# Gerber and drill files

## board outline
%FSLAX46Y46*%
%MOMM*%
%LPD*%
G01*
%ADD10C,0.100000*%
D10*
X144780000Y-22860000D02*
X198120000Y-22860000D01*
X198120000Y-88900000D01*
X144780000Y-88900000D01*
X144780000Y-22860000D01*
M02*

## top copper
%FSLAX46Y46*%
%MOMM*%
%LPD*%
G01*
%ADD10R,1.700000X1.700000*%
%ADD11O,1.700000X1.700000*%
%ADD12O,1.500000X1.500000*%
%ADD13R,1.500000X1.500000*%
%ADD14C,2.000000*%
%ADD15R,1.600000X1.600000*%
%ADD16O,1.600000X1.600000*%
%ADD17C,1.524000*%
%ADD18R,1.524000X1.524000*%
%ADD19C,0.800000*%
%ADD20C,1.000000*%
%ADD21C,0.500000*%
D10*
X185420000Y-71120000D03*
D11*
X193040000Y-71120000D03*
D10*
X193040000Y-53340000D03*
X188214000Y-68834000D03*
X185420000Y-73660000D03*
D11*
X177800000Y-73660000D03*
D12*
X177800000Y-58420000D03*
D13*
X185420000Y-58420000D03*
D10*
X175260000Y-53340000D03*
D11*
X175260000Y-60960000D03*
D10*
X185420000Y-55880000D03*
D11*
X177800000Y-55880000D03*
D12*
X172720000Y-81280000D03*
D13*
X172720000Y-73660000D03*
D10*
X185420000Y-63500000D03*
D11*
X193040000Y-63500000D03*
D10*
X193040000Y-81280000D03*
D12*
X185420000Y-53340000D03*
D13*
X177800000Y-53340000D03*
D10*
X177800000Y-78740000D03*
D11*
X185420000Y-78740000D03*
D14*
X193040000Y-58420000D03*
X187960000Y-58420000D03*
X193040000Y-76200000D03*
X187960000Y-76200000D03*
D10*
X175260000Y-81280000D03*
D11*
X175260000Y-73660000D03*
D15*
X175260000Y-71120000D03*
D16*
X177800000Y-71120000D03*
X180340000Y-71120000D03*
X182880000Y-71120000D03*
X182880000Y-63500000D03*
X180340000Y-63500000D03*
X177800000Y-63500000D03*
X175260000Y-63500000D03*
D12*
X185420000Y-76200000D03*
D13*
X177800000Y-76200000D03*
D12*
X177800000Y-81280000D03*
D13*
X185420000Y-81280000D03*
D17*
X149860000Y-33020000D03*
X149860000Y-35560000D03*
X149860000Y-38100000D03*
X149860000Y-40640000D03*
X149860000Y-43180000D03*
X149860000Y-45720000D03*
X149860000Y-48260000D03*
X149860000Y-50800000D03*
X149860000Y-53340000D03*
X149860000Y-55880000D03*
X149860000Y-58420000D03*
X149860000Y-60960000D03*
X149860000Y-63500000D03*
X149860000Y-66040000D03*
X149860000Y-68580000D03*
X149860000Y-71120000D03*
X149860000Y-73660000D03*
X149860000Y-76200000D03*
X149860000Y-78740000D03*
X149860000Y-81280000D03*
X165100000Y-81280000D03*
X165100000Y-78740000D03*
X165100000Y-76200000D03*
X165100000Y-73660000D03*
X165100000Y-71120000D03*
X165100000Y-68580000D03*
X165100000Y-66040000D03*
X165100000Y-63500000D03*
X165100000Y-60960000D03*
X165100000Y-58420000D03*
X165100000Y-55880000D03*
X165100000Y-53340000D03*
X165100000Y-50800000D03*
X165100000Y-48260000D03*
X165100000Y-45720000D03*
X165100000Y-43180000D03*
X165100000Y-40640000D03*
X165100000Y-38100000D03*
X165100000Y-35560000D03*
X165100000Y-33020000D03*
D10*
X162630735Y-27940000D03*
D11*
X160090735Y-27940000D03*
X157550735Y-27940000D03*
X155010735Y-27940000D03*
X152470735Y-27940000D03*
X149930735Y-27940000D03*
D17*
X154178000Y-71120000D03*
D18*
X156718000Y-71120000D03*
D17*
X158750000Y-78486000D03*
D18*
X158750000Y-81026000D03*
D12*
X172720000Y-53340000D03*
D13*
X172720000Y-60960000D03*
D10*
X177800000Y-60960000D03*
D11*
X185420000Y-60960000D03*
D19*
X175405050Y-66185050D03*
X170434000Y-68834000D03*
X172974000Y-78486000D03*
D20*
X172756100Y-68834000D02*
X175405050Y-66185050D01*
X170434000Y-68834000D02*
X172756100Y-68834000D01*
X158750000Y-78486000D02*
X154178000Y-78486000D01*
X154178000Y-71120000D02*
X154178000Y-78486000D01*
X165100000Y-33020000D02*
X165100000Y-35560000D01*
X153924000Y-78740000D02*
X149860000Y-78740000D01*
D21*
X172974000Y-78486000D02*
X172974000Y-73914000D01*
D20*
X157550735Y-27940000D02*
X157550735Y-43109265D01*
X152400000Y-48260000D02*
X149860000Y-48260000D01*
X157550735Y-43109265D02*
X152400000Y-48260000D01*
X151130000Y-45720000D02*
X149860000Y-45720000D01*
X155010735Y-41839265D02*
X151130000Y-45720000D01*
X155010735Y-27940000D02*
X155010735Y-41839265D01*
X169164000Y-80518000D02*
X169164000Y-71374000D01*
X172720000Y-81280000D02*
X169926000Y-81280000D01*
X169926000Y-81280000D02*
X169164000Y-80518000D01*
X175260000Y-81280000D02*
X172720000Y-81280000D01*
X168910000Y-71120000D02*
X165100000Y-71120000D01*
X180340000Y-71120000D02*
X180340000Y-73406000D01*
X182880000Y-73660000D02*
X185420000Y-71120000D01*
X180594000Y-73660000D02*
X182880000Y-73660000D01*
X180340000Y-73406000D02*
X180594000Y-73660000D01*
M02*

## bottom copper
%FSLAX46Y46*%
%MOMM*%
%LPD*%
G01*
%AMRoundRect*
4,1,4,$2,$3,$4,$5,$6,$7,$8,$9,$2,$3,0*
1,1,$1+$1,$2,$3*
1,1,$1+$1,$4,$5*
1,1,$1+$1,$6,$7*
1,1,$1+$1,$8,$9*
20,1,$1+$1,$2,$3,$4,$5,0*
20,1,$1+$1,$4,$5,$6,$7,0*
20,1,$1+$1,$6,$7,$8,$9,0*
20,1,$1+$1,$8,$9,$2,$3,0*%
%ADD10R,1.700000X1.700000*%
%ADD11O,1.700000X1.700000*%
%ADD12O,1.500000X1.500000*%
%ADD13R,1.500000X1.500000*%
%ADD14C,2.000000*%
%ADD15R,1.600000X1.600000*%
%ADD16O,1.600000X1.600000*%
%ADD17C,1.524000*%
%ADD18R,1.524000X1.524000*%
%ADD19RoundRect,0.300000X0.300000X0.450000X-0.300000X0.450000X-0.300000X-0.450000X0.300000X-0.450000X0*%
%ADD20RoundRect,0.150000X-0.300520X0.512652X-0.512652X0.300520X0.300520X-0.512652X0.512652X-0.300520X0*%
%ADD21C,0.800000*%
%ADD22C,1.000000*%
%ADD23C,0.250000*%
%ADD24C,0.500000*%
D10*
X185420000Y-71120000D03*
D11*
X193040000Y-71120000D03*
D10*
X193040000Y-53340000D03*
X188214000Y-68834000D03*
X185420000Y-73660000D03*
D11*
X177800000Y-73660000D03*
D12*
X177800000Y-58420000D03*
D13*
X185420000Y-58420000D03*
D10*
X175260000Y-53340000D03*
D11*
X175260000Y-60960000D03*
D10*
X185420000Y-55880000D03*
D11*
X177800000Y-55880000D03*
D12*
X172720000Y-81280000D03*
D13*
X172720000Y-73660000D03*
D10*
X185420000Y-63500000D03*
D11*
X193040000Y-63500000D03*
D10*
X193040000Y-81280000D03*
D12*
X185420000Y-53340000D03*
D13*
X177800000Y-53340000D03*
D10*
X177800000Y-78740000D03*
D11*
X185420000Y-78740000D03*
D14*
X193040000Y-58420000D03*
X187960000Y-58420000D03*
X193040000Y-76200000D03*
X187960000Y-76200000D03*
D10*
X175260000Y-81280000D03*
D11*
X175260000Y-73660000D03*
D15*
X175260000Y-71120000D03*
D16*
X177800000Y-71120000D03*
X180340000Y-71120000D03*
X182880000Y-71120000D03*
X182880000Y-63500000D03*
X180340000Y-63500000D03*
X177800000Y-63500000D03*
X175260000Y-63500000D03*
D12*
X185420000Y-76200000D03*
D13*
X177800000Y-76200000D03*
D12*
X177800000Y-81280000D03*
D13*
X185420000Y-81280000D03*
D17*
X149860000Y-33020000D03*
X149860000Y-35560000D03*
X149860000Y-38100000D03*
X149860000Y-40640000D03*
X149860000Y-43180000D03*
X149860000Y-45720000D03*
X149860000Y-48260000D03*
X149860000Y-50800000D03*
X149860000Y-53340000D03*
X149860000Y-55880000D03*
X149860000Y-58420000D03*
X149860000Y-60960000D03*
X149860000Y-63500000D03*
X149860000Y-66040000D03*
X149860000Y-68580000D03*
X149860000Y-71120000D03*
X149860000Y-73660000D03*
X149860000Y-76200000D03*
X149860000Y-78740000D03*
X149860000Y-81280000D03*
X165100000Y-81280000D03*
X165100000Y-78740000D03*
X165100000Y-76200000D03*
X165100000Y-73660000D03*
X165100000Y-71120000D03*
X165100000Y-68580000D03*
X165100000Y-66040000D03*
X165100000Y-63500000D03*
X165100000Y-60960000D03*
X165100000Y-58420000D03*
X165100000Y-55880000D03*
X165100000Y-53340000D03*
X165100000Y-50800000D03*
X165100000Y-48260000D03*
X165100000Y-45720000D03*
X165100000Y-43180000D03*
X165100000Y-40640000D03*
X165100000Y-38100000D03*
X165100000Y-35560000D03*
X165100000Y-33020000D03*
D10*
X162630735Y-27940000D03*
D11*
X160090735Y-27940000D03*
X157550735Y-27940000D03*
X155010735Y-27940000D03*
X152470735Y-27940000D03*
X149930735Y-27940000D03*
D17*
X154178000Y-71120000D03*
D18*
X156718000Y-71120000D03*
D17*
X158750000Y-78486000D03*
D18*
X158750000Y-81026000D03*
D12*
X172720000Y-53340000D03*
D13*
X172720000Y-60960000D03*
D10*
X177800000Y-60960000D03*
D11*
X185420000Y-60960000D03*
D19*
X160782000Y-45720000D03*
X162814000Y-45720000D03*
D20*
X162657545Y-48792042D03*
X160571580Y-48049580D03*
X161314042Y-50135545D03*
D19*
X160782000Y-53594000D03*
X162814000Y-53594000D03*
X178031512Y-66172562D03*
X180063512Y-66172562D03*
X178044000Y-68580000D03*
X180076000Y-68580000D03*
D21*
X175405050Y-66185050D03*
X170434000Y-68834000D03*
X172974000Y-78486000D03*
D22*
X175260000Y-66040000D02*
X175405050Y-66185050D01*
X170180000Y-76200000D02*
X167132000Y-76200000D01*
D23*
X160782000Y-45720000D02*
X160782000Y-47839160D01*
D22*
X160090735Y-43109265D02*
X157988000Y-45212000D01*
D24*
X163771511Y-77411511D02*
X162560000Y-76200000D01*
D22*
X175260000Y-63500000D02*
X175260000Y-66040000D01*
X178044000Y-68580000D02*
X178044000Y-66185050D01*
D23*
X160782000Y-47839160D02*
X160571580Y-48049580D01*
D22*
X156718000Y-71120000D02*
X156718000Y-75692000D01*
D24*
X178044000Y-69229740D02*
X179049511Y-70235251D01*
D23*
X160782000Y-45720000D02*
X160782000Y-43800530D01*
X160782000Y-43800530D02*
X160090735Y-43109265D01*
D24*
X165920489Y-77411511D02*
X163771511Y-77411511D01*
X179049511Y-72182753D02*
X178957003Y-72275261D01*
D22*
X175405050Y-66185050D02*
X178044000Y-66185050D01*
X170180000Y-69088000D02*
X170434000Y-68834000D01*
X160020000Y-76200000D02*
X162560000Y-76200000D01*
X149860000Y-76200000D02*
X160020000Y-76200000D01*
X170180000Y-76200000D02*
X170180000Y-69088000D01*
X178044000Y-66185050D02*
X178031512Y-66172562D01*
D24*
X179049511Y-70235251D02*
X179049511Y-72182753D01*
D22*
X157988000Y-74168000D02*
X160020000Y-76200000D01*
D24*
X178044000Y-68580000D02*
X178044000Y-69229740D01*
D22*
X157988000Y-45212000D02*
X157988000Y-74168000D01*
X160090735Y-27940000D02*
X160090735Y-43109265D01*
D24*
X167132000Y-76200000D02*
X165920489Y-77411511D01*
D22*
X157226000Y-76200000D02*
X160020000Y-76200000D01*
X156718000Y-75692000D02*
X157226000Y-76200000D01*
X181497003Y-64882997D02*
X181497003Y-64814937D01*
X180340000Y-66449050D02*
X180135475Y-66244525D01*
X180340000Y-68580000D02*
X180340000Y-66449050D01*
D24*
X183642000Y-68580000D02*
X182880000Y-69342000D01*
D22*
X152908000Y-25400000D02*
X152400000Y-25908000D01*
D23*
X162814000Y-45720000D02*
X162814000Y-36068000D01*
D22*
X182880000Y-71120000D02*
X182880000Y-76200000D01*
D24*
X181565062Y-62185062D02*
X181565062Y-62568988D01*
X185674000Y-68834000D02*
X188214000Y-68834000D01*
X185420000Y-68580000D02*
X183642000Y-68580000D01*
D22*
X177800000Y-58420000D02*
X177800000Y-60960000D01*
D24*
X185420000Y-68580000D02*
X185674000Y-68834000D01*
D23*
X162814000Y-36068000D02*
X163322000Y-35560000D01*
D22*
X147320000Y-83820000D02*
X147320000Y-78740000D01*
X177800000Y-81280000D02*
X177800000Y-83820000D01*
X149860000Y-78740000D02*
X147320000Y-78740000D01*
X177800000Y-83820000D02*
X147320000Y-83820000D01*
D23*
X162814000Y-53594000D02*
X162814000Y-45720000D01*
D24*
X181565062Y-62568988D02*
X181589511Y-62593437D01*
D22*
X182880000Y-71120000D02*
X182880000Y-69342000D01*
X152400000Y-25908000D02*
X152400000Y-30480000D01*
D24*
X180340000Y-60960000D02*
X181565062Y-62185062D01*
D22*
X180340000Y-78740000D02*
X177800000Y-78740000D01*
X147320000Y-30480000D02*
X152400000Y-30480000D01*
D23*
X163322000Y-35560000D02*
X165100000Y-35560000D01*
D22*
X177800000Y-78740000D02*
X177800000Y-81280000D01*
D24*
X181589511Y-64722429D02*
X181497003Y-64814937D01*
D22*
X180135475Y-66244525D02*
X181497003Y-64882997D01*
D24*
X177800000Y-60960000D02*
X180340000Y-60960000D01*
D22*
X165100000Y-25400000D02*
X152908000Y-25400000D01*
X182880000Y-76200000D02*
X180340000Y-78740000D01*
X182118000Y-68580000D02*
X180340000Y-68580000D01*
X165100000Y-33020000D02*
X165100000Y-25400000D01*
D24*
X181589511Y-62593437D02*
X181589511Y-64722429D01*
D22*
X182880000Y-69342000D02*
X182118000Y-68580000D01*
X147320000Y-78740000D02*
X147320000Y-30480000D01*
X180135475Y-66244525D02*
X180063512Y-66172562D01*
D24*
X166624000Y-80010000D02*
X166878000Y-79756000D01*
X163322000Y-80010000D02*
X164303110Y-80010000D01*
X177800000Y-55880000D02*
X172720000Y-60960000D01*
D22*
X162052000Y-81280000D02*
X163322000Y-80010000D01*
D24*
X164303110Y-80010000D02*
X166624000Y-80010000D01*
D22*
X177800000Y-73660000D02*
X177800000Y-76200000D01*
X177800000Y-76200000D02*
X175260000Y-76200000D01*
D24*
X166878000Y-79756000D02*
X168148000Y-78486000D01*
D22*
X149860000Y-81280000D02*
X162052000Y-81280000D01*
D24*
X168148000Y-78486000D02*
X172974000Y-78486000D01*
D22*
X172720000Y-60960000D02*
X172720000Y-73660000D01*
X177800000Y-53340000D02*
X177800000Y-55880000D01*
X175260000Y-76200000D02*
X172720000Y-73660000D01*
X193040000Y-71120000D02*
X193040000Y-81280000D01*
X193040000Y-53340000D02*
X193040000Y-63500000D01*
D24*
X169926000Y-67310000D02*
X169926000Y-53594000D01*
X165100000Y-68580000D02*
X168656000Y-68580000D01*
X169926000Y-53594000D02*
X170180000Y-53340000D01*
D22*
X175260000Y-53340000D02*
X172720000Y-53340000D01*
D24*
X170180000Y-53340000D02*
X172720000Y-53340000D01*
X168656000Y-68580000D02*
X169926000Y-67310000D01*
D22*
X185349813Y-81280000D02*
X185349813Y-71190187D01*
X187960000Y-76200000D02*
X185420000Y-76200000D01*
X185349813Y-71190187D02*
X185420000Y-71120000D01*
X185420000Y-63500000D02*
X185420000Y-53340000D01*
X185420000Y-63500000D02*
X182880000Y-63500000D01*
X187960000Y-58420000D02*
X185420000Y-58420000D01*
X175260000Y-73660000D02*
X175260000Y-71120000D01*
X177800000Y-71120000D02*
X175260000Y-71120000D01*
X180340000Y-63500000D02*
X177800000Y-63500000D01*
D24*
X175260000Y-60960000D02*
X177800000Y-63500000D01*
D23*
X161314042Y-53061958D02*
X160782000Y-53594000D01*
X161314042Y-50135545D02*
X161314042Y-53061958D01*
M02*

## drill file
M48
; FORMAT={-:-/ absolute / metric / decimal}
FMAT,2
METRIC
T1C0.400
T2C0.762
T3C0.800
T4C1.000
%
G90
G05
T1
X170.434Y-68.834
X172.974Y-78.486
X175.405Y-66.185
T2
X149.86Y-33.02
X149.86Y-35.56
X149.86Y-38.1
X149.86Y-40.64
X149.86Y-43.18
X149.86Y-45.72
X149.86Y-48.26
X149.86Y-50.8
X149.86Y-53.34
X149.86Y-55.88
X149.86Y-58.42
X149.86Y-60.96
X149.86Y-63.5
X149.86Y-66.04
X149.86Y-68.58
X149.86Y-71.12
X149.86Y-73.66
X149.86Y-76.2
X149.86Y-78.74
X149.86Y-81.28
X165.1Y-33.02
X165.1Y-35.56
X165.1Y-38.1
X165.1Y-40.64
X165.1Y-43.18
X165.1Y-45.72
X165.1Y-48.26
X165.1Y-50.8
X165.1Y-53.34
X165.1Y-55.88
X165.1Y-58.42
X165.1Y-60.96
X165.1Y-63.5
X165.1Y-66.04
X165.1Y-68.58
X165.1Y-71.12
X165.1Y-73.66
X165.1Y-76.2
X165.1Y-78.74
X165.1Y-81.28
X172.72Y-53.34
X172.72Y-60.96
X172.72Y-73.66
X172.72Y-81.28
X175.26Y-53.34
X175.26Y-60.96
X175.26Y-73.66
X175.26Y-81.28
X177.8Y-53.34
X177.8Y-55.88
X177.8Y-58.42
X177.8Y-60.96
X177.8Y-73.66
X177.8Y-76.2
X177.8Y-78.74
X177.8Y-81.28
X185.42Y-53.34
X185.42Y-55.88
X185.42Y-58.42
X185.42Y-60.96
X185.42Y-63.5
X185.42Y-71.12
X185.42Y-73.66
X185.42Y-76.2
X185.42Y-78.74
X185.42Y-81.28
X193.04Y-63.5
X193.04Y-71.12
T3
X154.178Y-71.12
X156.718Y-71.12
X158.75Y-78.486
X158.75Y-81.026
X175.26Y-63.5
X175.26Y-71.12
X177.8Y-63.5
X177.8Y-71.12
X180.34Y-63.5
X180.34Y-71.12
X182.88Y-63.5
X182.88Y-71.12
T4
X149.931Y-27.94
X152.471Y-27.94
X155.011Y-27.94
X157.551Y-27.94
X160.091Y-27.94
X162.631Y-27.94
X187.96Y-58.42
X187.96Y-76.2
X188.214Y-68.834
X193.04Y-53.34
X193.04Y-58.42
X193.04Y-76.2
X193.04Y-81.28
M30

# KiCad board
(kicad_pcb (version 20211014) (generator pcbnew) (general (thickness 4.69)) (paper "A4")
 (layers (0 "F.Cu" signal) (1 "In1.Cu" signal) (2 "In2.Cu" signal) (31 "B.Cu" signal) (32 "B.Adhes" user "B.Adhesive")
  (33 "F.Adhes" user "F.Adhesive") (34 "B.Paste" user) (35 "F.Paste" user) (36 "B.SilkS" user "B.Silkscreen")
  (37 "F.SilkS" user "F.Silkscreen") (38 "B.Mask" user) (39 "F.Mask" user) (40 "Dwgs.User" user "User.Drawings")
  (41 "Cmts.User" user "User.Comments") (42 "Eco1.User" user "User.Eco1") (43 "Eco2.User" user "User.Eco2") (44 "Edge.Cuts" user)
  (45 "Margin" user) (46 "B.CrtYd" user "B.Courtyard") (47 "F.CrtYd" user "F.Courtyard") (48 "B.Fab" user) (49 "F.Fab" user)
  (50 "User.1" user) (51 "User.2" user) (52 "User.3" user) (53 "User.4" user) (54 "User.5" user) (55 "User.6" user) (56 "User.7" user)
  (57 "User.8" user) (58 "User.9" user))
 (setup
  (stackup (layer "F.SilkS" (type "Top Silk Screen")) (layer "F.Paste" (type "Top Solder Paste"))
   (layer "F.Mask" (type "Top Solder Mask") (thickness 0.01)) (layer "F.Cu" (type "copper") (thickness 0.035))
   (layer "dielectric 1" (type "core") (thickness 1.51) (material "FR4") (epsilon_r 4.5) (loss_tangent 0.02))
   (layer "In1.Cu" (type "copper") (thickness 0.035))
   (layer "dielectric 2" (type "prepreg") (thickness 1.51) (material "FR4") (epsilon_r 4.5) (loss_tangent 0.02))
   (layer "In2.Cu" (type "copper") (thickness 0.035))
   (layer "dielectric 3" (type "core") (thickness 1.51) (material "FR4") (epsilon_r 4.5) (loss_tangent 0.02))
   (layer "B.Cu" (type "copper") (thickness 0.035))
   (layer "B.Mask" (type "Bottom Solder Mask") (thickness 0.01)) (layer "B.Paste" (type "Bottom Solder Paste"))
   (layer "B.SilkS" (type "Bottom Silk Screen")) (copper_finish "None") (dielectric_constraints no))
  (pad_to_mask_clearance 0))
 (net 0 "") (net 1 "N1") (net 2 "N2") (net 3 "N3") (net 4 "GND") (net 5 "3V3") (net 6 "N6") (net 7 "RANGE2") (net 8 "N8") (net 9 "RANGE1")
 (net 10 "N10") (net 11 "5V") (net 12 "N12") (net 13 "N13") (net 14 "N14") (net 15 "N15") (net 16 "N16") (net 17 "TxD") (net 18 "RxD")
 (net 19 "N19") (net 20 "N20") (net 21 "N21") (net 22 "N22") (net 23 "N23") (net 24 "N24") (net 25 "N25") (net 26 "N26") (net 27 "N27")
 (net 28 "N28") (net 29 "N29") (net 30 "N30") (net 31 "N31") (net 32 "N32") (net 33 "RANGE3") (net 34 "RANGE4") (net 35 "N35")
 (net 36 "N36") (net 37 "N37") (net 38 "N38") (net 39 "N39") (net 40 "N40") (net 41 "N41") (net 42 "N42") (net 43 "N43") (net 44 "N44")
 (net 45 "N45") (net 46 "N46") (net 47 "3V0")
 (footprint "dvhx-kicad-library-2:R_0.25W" (layer "F.Cu") (at 185.42 71.12)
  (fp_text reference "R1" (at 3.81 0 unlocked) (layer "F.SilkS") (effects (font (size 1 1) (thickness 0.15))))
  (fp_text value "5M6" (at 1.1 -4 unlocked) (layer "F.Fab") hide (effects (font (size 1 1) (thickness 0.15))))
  (pad "1" thru_hole rect (at 0 0 90) (size 1.7 1.7) (drill 0.762) (layers *.Cu *.Mask) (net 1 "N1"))
  (pad "2" thru_hole oval (at 7.62 0 90) (size 1.7 1.7) (drill 0.762) (layers *.Cu *.Mask) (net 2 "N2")))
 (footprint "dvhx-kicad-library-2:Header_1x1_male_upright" (layer "F.Cu") (at 193.04 53.34 -90)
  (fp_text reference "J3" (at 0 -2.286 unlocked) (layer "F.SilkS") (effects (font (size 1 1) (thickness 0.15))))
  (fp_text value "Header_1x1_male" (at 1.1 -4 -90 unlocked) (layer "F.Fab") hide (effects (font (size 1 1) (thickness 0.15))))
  (pad "1" thru_hole rect (at 0 0 270) (size 1.7 1.7) (drill 1) (layers *.Cu *.Mask) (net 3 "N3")))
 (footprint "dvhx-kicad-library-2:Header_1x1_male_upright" (layer "F.Cu") (at 188.214 68.834)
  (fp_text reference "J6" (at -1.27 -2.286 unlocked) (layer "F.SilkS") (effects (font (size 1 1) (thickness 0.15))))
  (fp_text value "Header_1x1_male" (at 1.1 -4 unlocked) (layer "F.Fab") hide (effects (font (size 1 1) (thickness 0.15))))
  (pad "1" thru_hole rect (at 0 0) (size 1.7 1.7) (drill 1) (layers *.Cu *.Mask) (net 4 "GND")))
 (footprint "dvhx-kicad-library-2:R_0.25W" (layer "F.Cu") (at 185.42 73.66 180)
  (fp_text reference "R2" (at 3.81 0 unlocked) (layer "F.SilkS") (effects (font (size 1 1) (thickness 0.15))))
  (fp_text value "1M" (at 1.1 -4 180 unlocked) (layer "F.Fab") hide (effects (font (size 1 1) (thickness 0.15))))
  (pad "1" thru_hole rect (at 0 0 270) (size 1.7 1.7) (drill 0.762) (layers *.Cu *.Mask) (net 1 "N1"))
  (pad "2" thru_hole oval (at 7.62 0 270) (size 1.7 1.7) (drill 0.762) (layers *.Cu *.Mask) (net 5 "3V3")))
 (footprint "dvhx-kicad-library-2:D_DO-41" (layer "F.Cu") (at 181.61 58.42 90)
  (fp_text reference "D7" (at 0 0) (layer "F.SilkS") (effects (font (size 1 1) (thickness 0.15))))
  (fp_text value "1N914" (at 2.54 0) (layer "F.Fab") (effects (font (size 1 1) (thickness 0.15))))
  (pad "A" thru_hole oval (at 0 -3.81 180) (size 1.5 1.5) (drill 0.762) (layers *.Cu *.Mask) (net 4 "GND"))
  (pad "K" thru_hole rect (at 0 3.81 180) (size 1.5 1.5) (drill 0.762) (layers *.Cu *.Mask) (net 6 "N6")))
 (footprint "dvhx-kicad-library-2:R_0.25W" (layer "F.Cu") (at 175.26 53.34 -90)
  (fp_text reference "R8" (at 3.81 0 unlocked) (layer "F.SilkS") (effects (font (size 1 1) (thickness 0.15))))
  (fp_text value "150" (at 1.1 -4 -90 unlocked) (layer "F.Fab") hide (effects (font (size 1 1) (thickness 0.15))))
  (pad "1" thru_hole rect (at 0 0) (size 1.7 1.7) (drill 0.762) (layers *.Cu *.Mask) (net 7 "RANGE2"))
  (pad "2" thru_hole oval (at 7.62 0) (size 1.7 1.7) (drill 0.762) (layers *.Cu *.Mask) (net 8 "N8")))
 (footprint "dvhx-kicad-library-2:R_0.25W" (layer "F.Cu") (at 185.42 55.88 180)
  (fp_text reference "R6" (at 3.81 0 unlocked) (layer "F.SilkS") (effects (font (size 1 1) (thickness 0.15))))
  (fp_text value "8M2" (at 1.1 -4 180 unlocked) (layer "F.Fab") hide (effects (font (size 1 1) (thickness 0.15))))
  (pad "1" thru_hole rect (at 0 0 270) (size 1.7 1.7) (drill 0.762) (layers *.Cu *.Mask) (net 6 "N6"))
  (pad "2" thru_hole oval (at 7.62 0 270) (size 1.7 1.7) (drill 0.762) (layers *.Cu *.Mask) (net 5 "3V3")))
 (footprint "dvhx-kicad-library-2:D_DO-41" (layer "F.Cu") (at 172.72 77.47 180)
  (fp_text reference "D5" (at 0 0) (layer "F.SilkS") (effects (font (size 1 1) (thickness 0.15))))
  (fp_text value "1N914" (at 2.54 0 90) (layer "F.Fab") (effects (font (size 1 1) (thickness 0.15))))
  (pad "A" thru_hole oval (at 0 -3.81 270) (size 1.5 1.5) (drill 0.762) (layers *.Cu *.Mask) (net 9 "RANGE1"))
  (pad "K" thru_hole rect (at 0 3.81 270) (size 1.5 1.5) (drill 0.762) (layers *.Cu *.Mask) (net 5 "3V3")))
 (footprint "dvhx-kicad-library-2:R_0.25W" (layer "F.Cu") (at 185.42 63.5)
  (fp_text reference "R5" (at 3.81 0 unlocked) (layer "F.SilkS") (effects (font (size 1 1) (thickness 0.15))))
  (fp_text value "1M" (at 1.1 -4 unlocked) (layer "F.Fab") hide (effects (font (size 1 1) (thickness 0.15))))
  (pad "1" thru_hole rect (at 0 0 90) (size 1.7 1.7) (drill 0.762) (layers *.Cu *.Mask) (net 6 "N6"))
  (pad "2" thru_hole oval (at 7.62 0 90) (size 1.7 1.7) (drill 0.762) (layers *.Cu *.Mask) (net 3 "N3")))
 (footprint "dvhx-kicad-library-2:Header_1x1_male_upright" (layer "F.Cu") (at 193.04 81.28 -90)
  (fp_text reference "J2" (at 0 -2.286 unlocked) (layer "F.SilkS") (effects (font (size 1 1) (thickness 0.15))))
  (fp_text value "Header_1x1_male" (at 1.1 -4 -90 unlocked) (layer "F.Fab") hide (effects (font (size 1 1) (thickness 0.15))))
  (pad "1" thru_hole rect (at 0 0 270) (size 1.7 1.7) (drill 1) (layers *.Cu *.Mask) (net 2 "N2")))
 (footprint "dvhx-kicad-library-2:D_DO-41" (layer "F.Cu") (at 181.61 53.34 -90)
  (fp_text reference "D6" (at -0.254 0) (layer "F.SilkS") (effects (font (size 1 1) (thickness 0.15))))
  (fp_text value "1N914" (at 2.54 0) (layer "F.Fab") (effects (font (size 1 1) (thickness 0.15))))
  (pad "A" thru_hole oval (at 0 -3.81) (size 1.5 1.5) (drill 0.762) (layers *.Cu *.Mask) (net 6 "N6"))
  (pad "K" thru_hole rect (at 0 3.81) (size 1.5 1.5) (drill 0.762) (layers *.Cu *.Mask) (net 5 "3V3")))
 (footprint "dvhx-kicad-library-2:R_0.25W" (layer "F.Cu") (at 177.8 78.74)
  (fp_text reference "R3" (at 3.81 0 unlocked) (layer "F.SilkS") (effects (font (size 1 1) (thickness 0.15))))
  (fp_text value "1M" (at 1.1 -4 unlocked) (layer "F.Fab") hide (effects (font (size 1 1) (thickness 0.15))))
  (pad "1" thru_hole rect (at 0 0 90) (size 1.7 1.7) (drill 0.762) (layers *.Cu *.Mask) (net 4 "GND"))
  (pad "2" thru_hole oval (at 7.62 0 90) (size 1.7 1.7) (drill 0.762) (layers *.Cu *.Mask) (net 1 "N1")))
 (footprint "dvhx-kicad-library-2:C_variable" (layer "F.Cu") (at 193.04 58.42 -90)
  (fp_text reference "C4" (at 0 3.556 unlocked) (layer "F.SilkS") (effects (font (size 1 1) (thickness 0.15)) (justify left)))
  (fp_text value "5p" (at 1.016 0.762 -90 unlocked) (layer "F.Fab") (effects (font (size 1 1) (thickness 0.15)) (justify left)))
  (pad "1" thru_hole circle (at 0 0 270) (size 2 2) (drill 1) (layers *.Cu *.Mask) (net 3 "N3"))
  (pad "2" thru_hole circle (at 0 5.08 270) (size 2 2) (drill 1) (layers *.Cu *.Mask) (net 6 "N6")))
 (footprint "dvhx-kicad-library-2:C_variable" (layer "F.Cu") (at 193.04 76.2 -90)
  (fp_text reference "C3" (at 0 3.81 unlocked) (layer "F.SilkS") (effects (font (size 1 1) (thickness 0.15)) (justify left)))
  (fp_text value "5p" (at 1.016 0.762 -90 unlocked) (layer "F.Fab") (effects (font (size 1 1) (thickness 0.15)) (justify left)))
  (pad "1" thru_hole circle (at 0 0 270) (size 2 2) (drill 1) (layers *.Cu *.Mask) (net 2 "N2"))
  (pad "2" thru_hole circle (at 0 5.08 270) (size 2 2) (drill 1) (layers *.Cu *.Mask) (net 1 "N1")))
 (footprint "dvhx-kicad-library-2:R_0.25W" (layer "F.Cu") (at 175.26 81.28 90)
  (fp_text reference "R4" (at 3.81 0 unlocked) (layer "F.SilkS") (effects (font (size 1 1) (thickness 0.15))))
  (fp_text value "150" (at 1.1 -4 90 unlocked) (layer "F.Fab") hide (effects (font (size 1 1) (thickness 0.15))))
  (pad "1" thru_hole rect (at 0 0 180) (size 1.7 1.7) (drill 0.762) (layers *.Cu *.Mask) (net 9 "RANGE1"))
  (pad "2" thru_hole oval (at 7.62 0 180) (size 1.7 1.7) (drill 0.762) (layers *.Cu *.Mask) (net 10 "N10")))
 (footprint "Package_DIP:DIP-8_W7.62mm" (layer "F.Cu") (at 175.26 71.12 90)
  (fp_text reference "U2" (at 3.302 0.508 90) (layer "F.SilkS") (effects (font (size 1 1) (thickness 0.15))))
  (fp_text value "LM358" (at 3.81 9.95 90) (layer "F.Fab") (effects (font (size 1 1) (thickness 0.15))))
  (pad "1" thru_hole rect (at 0 0 90) (size 1.6 1.6) (drill 0.8) (layers *.Cu *.Mask) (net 10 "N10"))
  (pad "2" thru_hole oval (at 0 2.54 90) (size 1.6 1.6) (drill 0.8) (layers *.Cu *.Mask) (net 10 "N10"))
  (pad "3" thru_hole oval (at 0 5.08 90) (size 1.6 1.6) (drill 0.8) (layers *.Cu *.Mask) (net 1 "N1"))
  (pad "4" thru_hole oval (at 0 7.62 90) (size 1.6 1.6) (drill 0.8) (layers *.Cu *.Mask) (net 4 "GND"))
  (pad "5" thru_hole oval (at 7.62 7.62 90) (size 1.6 1.6) (drill 0.8) (layers *.Cu *.Mask) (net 6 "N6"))
  (pad "6" thru_hole oval (at 7.62 5.08 90) (size 1.6 1.6) (drill 0.8) (layers *.Cu *.Mask) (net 8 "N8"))
  (pad "7" thru_hole oval (at 7.62 2.54 90) (size 1.6 1.6) (drill 0.8) (layers *.Cu *.Mask) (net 8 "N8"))
  (pad "8" thru_hole oval (at 7.62 0 90) (size 1.6 1.6) (drill 0.8) (layers *.Cu *.Mask) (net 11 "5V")))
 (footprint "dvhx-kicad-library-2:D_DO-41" (layer "F.Cu") (at 181.61 76.2 -90)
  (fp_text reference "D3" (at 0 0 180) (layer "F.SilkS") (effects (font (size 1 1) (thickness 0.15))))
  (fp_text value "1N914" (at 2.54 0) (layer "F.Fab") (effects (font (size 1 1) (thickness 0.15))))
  (pad "A" thru_hole oval (at 0 -3.81) (size 1.5 1.5) (drill 0.762) (layers *.Cu *.Mask) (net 1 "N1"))
  (pad "K" thru_hole rect (at 0 3.81) (size 1.5 1.5) (drill 0.762) (layers *.Cu *.Mask) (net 5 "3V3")))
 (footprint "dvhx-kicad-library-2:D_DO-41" (layer "F.Cu") (at 181.61 81.28 90)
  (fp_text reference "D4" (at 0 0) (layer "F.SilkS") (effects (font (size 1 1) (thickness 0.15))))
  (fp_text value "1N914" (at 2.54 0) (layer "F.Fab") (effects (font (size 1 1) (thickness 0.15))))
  (pad "A" thru_hole oval (at 0 -3.81 180) (size 1.5 1.5) (drill 0.762) (layers *.Cu *.Mask) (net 4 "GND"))
  (pad "K" thru_hole rect (at 0 3.81 180) (size 1.5 1.5) (drill 0.762) (layers *.Cu *.Mask) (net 1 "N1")))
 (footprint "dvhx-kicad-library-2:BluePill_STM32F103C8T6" (layer "F.Cu") (at 149.86 33.02)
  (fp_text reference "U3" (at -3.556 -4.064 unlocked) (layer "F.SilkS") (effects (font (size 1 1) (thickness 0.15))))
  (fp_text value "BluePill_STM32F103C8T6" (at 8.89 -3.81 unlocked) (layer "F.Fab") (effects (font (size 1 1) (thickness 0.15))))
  (pad "1" thru_hole circle (at 0 0) (size 1.524 1.524) (drill 0.762) (layers *.Cu *.Mask) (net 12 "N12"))
  (pad "2" thru_hole circle (at 0 2.54) (size 1.524 1.524) (drill 0.762) (layers *.Cu *.Mask) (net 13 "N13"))
  (pad "3" thru_hole circle (at 0 5.08) (size 1.524 1.524) (drill 0.762) (layers *.Cu *.Mask) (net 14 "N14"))
  (pad "4" thru_hole circle (at 0 7.62) (size 1.524 1.524) (drill 0.762) (layers *.Cu *.Mask) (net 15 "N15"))
  (pad "5" thru_hole circle (at 0 10.16) (size 1.524 1.524) (drill 0.762) (layers *.Cu *.Mask) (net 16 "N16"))
  (pad "6" thru_hole circle (at 0 12.7) (size 1.524 1.524) (drill 0.762) (layers *.Cu *.Mask) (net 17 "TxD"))
  (pad "7" thru_hole circle (at 0 15.24) (size 1.524 1.524) (drill 0.762) (layers *.Cu *.Mask) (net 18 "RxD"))
  (pad "8" thru_hole circle (at 0 17.78) (size 1.524 1.524) (drill 0.762) (layers *.Cu *.Mask) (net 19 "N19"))
  (pad "9" thru_hole circle (at 0 20.32) (size 1.524 1.524) (drill 0.762) (layers *.Cu *.Mask) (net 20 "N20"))
  (pad "10" thru_hole circle (at 0 22.86) (size 1.524 1.524) (drill 0.762) (layers *.Cu *.Mask) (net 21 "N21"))
  (pad "11" thru_hole circle (at 0 25.4) (size 1.524 1.524) (drill 0.762) (layers *.Cu *.Mask) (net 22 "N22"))
  (pad "12" thru_hole circle (at 0 27.94) (size 1.524 1.524) (drill 0.762) (layers *.Cu *.Mask) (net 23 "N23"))
  (pad "13" thru_hole circle (at 0 30.48) (size 1.524 1.524) (drill 0.762) (layers *.Cu *.Mask) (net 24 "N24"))
  (pad "14" thru_hole circle (at 0 33.02) (size 1.524 1.524) (drill 0.762) (layers *.Cu *.Mask) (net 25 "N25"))
  (pad "15" thru_hole circle (at 0 35.56) (size 1.524 1.524) (drill 0.762) (layers *.Cu *.Mask) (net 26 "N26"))
  (pad "16" thru_hole circle (at 0 38.1) (size 1.524 1.524) (drill 0.762) (layers *.Cu *.Mask) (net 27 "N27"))
  (pad "17" thru_hole circle (at 0 40.64) (size 1.524 1.524) (drill 0.762) (layers *.Cu *.Mask) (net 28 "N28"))
  (pad "18" thru_hole circle (at 0 43.18) (size 1.524 1.524) (drill 0.762) (layers *.Cu *.Mask) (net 11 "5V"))
  (pad "19" thru_hole circle (at 0 45.72) (size 1.524 1.524) (drill 0.762) (layers *.Cu *.Mask) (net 4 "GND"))
  (pad "20" thru_hole circle (at 0 48.26) (size 1.524 1.524) (drill 0.762) (layers *.Cu *.Mask) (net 5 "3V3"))
  (pad "21" thru_hole circle (at 15.24 48.26) (size 1.524 1.524) (drill 0.762) (layers *.Cu *.Mask) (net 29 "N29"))
  (pad "22" thru_hole circle (at 15.24 45.72) (size 1.524 1.524) (drill 0.762) (layers *.Cu *.Mask) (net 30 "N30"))
  (pad "23" thru_hole circle (at 15.24 43.18) (size 1.524 1.524) (drill 0.762) (layers *.Cu *.Mask) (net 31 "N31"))
  (pad "24" thru_hole circle (at 15.24 40.64) (size 1.524 1.524) (drill 0.762) (layers *.Cu *.Mask) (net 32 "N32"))
  (pad "25" thru_hole circle (at 15.24 38.1) (size 1.524 1.524) (drill 0.762) (layers *.Cu *.Mask) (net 9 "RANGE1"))
  (pad "26" thru_hole circle (at 15.24 35.56) (size 1.524 1.524) (drill 0.762) (layers *.Cu *.Mask) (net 7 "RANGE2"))
  (pad "27" thru_hole circle (at 15.24 33.02) (size 1.524 1.524) (drill 0.762) (layers *.Cu *.Mask) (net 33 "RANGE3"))
  (pad "28" thru_hole circle (at 15.24 30.48) (size 1.524 1.524) (drill 0.762) (layers *.Cu *.Mask) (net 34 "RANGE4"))
  (pad "29" thru_hole circle (at 15.24 27.94) (size 1.524 1.524) (drill 0.762) (layers *.Cu *.Mask) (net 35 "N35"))
  (pad "30" thru_hole circle (at 15.24 25.4) (size 1.524 1.524) (drill 0.762) (layers *.Cu *.Mask) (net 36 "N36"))
  (pad "31" thru_hole circle (at 15.24 22.86) (size 1.524 1.524) (drill 0.762) (layers *.Cu *.Mask) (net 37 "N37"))
  (pad "32" thru_hole circle (at 15.24 20.32) (size 1.524 1.524) (drill 0.762) (layers *.Cu *.Mask) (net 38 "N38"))
  (pad "33" thru_hole circle (at 15.24 17.78) (size 1.524 1.524) (drill 0.762) (layers *.Cu *.Mask) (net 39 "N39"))
  (pad "34" thru_hole circle (at 15.24 15.24) (size 1.524 1.524) (drill 0.762) (layers *.Cu *.Mask) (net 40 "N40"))
  (pad "35" thru_hole circle (at 15.24 12.7) (size 1.524 1.524) (drill 0.762) (layers *.Cu *.Mask) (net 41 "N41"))
  (pad "36" thru_hole circle (at 15.24 10.16) (size 1.524 1.524) (drill 0.762) (layers *.Cu *.Mask) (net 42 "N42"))
  (pad "37" thru_hole circle (at 15.24 7.62) (size 1.524 1.524) (drill 0.762) (layers *.Cu *.Mask) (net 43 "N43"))
  (pad "38" thru_hole circle (at 15.24 5.08) (size 1.524 1.524) (drill 0.762) (layers *.Cu *.Mask) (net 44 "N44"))
  (pad "39" thru_hole circle (at 15.24 2.54) (size 1.524 1.524) (drill 0.762) (layers *.Cu *.Mask) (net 4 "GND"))
  (pad "40" thru_hole circle (at 15.24 0) (size 1.524 1.524) (drill 0.762) (layers *.Cu *.Mask) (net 4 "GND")))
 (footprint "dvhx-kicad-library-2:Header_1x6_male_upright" (layer "F.Cu") (at 162.630735 27.94 180)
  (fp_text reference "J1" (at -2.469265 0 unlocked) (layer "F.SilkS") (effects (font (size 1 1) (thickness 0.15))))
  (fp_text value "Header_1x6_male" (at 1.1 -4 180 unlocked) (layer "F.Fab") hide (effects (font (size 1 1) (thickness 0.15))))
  (pad "1" thru_hole rect (at 0 0 270) (size 1.7 1.7) (drill 1) (layers *.Cu *.Mask) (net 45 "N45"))
  (pad "2" thru_hole oval (at 2.54 0 270) (size 1.7 1.7) (drill 1) (layers *.Cu *.Mask) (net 11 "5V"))
  (pad "3" thru_hole oval (at 5.08 0 270) (size 1.7 1.7) (drill 1) (layers *.Cu *.Mask) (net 18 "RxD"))
  (pad "4" thru_hole oval (at 7.62 0 270) (size 1.7 1.7) (drill 1) (layers *.Cu *.Mask) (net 17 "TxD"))
  (pad "5" thru_hole oval (at 10.16 0 270) (size 1.7 1.7) (drill 1) (layers *.Cu *.Mask) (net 4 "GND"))
  (pad "6" thru_hole oval (at 12.7 0 270) (size 1.7 1.7) (drill 1) (layers *.Cu *.Mask) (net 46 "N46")))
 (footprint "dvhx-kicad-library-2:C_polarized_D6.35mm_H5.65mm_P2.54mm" (layer "F.Cu") (at 155.448 71.12 -90)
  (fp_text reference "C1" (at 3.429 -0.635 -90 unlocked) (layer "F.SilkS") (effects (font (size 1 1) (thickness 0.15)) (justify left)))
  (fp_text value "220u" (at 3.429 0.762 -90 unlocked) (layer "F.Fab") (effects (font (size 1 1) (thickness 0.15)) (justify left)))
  (pad "N" thru_hole circle (at 0 1.27 180) (size 1.524 1.524) (drill 0.8) (layers *.Cu *.Mask) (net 4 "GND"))
  (pad "P" thru_hole rect (at 0 -1.27 180) (size 1.524 1.524) (drill 0.8) (layers *.Cu *.Mask) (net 11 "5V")))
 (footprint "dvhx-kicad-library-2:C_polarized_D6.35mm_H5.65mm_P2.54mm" (layer "F.Cu") (at 158.75 79.756 180)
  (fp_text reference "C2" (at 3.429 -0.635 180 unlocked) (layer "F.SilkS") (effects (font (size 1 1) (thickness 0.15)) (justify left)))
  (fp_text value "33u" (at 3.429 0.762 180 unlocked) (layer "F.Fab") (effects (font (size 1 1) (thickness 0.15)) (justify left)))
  (pad "N" thru_hole circle (at 0 1.27 90) (size 1.524 1.524) (drill 0.8) (layers *.Cu *.Mask) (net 4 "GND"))
  (pad "P" thru_hole rect (at 0 -1.27 90) (size 1.524 1.524) (drill 0.8) (layers *.Cu *.Mask) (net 5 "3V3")))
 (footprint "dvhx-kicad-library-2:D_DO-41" (layer "F.Cu") (at 172.72 57.15)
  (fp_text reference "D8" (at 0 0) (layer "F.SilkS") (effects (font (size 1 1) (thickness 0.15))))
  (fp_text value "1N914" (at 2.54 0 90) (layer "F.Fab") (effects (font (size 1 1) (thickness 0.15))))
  (pad "A" thru_hole oval (at 0 -3.81 90) (size 1.5 1.5) (drill 0.762) (layers *.Cu *.Mask) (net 7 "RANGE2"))
  (pad "K" thru_hole rect (at 0 3.81 90) (size 1.5 1.5) (drill 0.762) (layers *.Cu *.Mask) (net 5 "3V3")))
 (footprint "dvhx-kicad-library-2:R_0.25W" (layer "F.Cu") (at 177.8 60.96)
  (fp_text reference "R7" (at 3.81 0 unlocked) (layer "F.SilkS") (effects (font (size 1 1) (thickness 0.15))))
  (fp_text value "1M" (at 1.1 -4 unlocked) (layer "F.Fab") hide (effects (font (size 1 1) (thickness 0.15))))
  (pad "1" thru_hole rect (at 0 0 90) (size 1.7 1.7) (drill 0.762) (layers *.Cu *.Mask) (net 4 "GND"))
  (pad "2" thru_hole oval (at 7.62 0 90) (size 1.7 1.7) (drill 0.762) (layers *.Cu *.Mask) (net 6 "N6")))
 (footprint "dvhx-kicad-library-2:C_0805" (layer "B.Cu") (at 161.798 45.72 -90)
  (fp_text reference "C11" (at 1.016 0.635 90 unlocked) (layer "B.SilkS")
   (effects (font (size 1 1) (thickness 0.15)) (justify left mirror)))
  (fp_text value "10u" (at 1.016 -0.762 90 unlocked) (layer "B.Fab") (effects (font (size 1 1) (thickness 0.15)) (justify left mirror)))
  (pad "1" smd roundrect (at 0 1.016 180) (size 1.2 1.5) (layers "B.Cu" "B.Paste" "B.Mask") (roundrect_rratio 0.25) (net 11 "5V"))
  (pad "2" smd roundrect (at 0 -1.016 180) (size 1.2 1.5) (layers "B.Cu" "B.Paste" "B.Mask") (roundrect_rratio 0.25) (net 4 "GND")))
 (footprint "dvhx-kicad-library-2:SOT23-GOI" (layer "B.Cu") (at 161.29 48.768 -135)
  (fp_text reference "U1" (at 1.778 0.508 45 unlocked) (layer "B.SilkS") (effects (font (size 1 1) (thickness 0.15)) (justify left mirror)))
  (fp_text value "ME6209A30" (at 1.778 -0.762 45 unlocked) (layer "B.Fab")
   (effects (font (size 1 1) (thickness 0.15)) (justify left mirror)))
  (pad "G" smd roundrect (at -0.95 -0.984 225) (size 0.6 1.45) (layers "B.Cu" "B.Paste" "B.Mask") (roundrect_rratio 0.25) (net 4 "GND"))
  (pad "I" smd roundrect (at 0 1.016 225) (size 0.6 1.45) (layers "B.Cu" "B.Paste" "B.Mask") (roundrect_rratio 0.25) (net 11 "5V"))
  (pad "O" smd roundrect (at 0.95 -0.984 225) (size 0.6 1.45) (layers "B.Cu" "B.Paste" "B.Mask") (roundrect_rratio 0.25) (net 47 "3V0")))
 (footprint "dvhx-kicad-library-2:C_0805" (layer "B.Cu") (at 161.798 53.594 -90)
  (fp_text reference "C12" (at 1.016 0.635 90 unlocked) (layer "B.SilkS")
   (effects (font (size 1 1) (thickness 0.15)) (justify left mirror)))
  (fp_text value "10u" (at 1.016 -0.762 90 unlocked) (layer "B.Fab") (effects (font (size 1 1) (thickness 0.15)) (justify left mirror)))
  (pad "1" smd roundrect (at 0 1.016 180) (size 1.2 1.5) (layers "B.Cu" "B.Paste" "B.Mask") (roundrect_rratio 0.25) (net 47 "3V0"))
  (pad "2" smd roundrect (at 0 -1.016 180) (size 1.2 1.5) (layers "B.Cu" "B.Paste" "B.Mask") (roundrect_rratio 0.25) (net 4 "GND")))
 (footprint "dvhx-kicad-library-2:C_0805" (layer "B.Cu") (at 179.047512 66.172562 -90)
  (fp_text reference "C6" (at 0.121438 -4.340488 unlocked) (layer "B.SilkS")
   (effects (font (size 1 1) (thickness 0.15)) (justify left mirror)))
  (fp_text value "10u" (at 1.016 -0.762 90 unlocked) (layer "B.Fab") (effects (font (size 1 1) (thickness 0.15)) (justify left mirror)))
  (pad "1" smd roundrect (at 0 1.016 180) (size 1.2 1.5) (layers "B.Cu" "B.Paste" "B.Mask") (roundrect_rratio 0.25) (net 11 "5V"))
  (pad "2" smd roundrect (at 0 -1.016 180) (size 1.2 1.5) (layers "B.Cu" "B.Paste" "B.Mask") (roundrect_rratio 0.25) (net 4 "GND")))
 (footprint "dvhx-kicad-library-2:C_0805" (layer "B.Cu") (at 179.06 68.58 -90)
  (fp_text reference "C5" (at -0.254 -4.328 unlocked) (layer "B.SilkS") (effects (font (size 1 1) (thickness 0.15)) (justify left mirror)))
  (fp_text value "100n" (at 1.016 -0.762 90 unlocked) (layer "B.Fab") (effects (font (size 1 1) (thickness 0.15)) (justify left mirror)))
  (pad "1" smd roundrect (at 0 1.016 180) (size 1.2 1.5) (layers "B.Cu" "B.Paste" "B.Mask") (roundrect_rratio 0.25) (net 11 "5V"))
  (pad "2" smd roundrect (at 0 -1.016 180) (size 1.2 1.5) (layers "B.Cu" "B.Paste" "B.Mask") (roundrect_rratio 0.25) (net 4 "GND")))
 (gr_rect (start 144.78 22.86) (end 198.12 88.9) (layer "Edge.Cuts") (width 0.1) (fill none))
 (segment (start 172.7561 68.834) (end 175.40505 66.18505) (width 1) (layer "F.Cu") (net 11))
 (segment (start 170.434 68.834) (end 172.7561 68.834) (width 1) (layer "F.Cu") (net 11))
 (via (at 175.40505 66.18505) (size 0.8) (drill 0.4) (layers "F.Cu" "B.Cu") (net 11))
 (via (at 170.434 68.834) (size 0.8) (drill 0.4) (layers "F.Cu" "B.Cu") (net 11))
 (segment (start 175.26 66.04) (end 175.40505 66.18505) (width 1) (layer "B.Cu") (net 11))
 (segment (start 170.18 76.2) (end 167.132 76.2) (width 1) (layer "B.Cu") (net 11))
 (segment (start 160.782 45.72) (end 160.782 47.83916) (width 0.25) (layer "B.Cu") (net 11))
 (segment (start 160.090735 43.109265) (end 157.988 45.212) (width 1) (layer "B.Cu") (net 11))
 (segment (start 163.771511 77.411511) (end 162.56 76.2) (width 0.5) (layer "B.Cu") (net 11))
 (segment (start 175.26 63.5) (end 175.26 66.04) (width 1) (layer "B.Cu") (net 11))
 (segment (start 178.044 68.58) (end 178.044 66.18505) (width 1) (layer "B.Cu") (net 11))
 (segment (start 160.782 47.83916) (end 160.57158 48.04958) (width 0.25) (layer "B.Cu") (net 11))
 (segment (start 156.718 71.12) (end 156.718 75.692) (width 1) (layer "B.Cu") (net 11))
 (segment (start 178.044 69.22974) (end 179.049511 70.235251) (width 0.5) (layer "B.Cu") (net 11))
 (segment (start 160.782 45.72) (end 160.782 43.80053) (width 0.25) (layer "B.Cu") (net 11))
 (segment (start 160.782 43.80053) (end 160.090735 43.109265) (width 0.25) (layer "B.Cu") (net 11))
 (segment (start 165.920489 77.411511) (end 163.771511 77.411511) (width 0.5) (layer "B.Cu") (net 11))
 (segment (start 179.049511 72.182753) (end 178.957003 72.275261) (width 0.5) (layer "B.Cu") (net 11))
 (segment (start 175.40505 66.18505) (end 178.044 66.18505) (width 1) (layer "B.Cu") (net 11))
 (segment (start 170.18 69.088) (end 170.434 68.834) (width 1) (layer "B.Cu") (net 11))
 (segment (start 160.02 76.2) (end 162.56 76.2) (width 1) (layer "B.Cu") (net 11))
 (segment (start 149.86 76.2) (end 160.02 76.2) (width 1) (layer "B.Cu") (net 11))
 (segment (start 170.18 76.2) (end 170.18 69.088) (width 1) (layer "B.Cu") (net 11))
 (segment (start 178.044 66.18505) (end 178.031512 66.172562) (width 1) (layer "B.Cu") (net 11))
 (segment (start 179.049511 70.235251) (end 179.049511 72.182753) (width 0.5) (layer "B.Cu") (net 11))
 (segment (start 157.988 74.168) (end 160.02 76.2) (width 1) (layer "B.Cu") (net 11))
 (segment (start 178.044 68.58) (end 178.044 69.22974) (width 0.5) (layer "B.Cu") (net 11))
 (segment (start 157.988 45.212) (end 157.988 74.168) (width 1) (layer "B.Cu") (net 11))
 (segment (start 160.090735 27.94) (end 160.090735 43.109265) (width 1) (layer "B.Cu") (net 11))
 (segment (start 167.132 76.2) (end 165.920489 77.411511) (width 0.5) (layer "B.Cu") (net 11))
 (segment (start 157.226 76.2) (end 160.02 76.2) (width 1) (layer "B.Cu") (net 11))
 (segment (start 156.718 75.692) (end 157.226 76.2) (width 1) (layer "B.Cu") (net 11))
 (segment (start 158.75 78.486) (end 154.178 78.486) (width 1) (layer "F.Cu") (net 4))
 (segment (start 154.178 71.12) (end 154.178 78.486) (width 1) (layer "F.Cu") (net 4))
 (segment (start 165.1 33.02) (end 165.1 35.56) (width 1) (layer "F.Cu") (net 4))
 (segment (start 153.924 78.74) (end 149.86 78.74) (width 1) (layer "F.Cu") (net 4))
 (segment (start 181.497003 64.882997) (end 181.497003 64.814937) (width 1) (layer "B.Cu") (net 4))
 (segment (start 180.34 66.44905) (end 180.135475 66.244525) (width 1) (layer "B.Cu") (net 4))
 (segment (start 180.34 68.58) (end 180.34 66.44905) (width 1) (layer "B.Cu") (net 4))
 (segment (start 183.642 68.58) (end 182.88 69.342) (width 0.5) (layer "B.Cu") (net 4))
 (segment (start 152.908 25.4) (end 152.4 25.908) (width 1) (layer "B.Cu") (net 4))
 (segment (start 162.814 45.72) (end 162.814 36.068) (width 0.25) (layer "B.Cu") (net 4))
 (segment (start 182.88 71.12) (end 182.88 76.2) (width 1) (layer "B.Cu") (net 4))
 (segment (start 181.565062 62.185062) (end 181.565062 62.568988) (width 0.5) (layer "B.Cu") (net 4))
 (segment (start 185.674 68.834) (end 188.214 68.834) (width 0.5) (layer "B.Cu") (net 4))
 (segment (start 185.42 68.58) (end 183.642 68.58) (width 0.5) (layer "B.Cu") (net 4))
 (segment (start 177.8 58.42) (end 177.8 60.96) (width 1) (layer "B.Cu") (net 4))
 (segment (start 185.42 68.58) (end 185.674 68.834) (width 0.5) (layer "B.Cu") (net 4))
 (segment (start 162.814 36.068) (end 163.322 35.56) (width 0.25) (layer "B.Cu") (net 4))
 (segment (start 147.32 83.82) (end 147.32 78.74) (width 1) (layer "B.Cu") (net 4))
 (segment (start 177.8 81.28) (end 177.8 83.82) (width 1) (layer "B.Cu") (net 4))
 (segment (start 149.86 78.74) (end 147.32 78.74) (width 1) (layer "B.Cu") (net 4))
 (segment (start 177.8 83.82) (end 147.32 83.82) (width 1) (layer "B.Cu") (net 4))
 (segment (start 162.814 53.594) (end 162.814 45.72) (width 0.25) (layer "B.Cu") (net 4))
 (segment (start 181.565062 62.568988) (end 181.589511 62.593437) (width 0.5) (layer "B.Cu") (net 4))
 (segment (start 182.88 71.12) (end 182.88 69.342) (width 1) (layer "B.Cu") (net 4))
 (segment (start 152.4 25.908) (end 152.4 30.48) (width 1) (layer "B.Cu") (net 4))
 (segment (start 180.34 60.96) (end 181.565062 62.185062) (width 0.5) (layer "B.Cu") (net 4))
 (segment (start 180.34 78.74) (end 177.8 78.74) (width 1) (layer "B.Cu") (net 4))
 (segment (start 147.32 30.48) (end 152.4 30.48) (width 1) (layer "B.Cu") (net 4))
 (segment (start 163.322 35.56) (end 165.1 35.56) (width 0.25) (layer "B.Cu") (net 4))
 (segment (start 177.8 78.74) (end 177.8 81.28) (width 1) (layer "B.Cu") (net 4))
 (segment (start 181.589511 64.722429) (end 181.497003 64.814937) (width 0.5) (layer "B.Cu") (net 4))
 (segment (start 180.135475 66.244525) (end 181.497003 64.882997) (width 1) (layer "B.Cu") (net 4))
 (segment (start 177.8 60.96) (end 180.34 60.96) (width 0.5) (layer "B.Cu") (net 4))
 (segment (start 165.1 25.4) (end 152.908 25.4) (width 1) (layer "B.Cu") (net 4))
 (segment (start 182.88 76.2) (end 180.34 78.74) (width 1) (layer "B.Cu") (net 4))
 (segment (start 182.118 68.58) (end 180.34 68.58) (width 1) (layer "B.Cu") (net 4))
 (segment (start 165.1 33.02) (end 165.1 25.4) (width 1) (layer "B.Cu") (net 4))
 (segment (start 181.589511 62.593437) (end 181.589511 64.722429) (width 0.5) (layer "B.Cu") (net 4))
 (segment (start 182.88 69.342) (end 182.118 68.58) (width 1) (layer "B.Cu") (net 4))
 (segment (start 147.32 78.74) (end 147.32 30.48) (width 1) (layer "B.Cu") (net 4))
 (segment (start 180.135475 66.244525) (end 180.063512 66.172562) (width 1) (layer "B.Cu") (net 4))
 (segment (start 172.974 78.486) (end 172.974 73.914) (width 0.5) (layer "F.Cu") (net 5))
 (via (at 172.974 78.486) (size 0.8) (drill 0.4) (layers "F.Cu" "B.Cu") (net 5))
 (segment (start 166.624 80.01) (end 166.878 79.756) (width 0.5) (layer "B.Cu") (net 5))
 (segment (start 163.322 80.01) (end 164.30311 80.01) (width 0.5) (layer "B.Cu") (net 5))
 (segment (start 177.8 55.88) (end 172.72 60.96) (width 0.5) (layer "B.Cu") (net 5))
 (segment (start 162.052 81.28) (end 163.322 80.01) (width 1) (layer "B.Cu") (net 5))
 (segment (start 164.30311 80.01) (end 166.624 80.01) (width 0.5) (layer "B.Cu") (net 5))
 (segment (start 177.8 73.66) (end 177.8 76.2) (width 1) (layer "B.Cu") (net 5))
 (segment (start 177.8 76.2) (end 175.26 76.2) (width 1) (layer "B.Cu") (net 5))
 (segment (start 166.878 79.756) (end 168.148 78.486) (width 0.5) (layer "B.Cu") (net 5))
 (segment (start 149.86 81.28) (end 162.052 81.28) (width 1) (layer "B.Cu") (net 5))
 (segment (start 168.148 78.486) (end 172.974 78.486) (width 0.5) (layer "B.Cu") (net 5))
 (segment (start 172.72 60.96) (end 172.72 73.66) (width 1) (layer "B.Cu") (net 5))
 (segment (start 177.8 53.34) (end 177.8 55.88) (width 1) (layer "B.Cu") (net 5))
 (segment (start 175.26 76.2) (end 172.72 73.66) (width 1) (layer "B.Cu") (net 5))
 (segment (start 157.550735 27.94) (end 157.550735 43.109265) (width 1) (layer "F.Cu") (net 18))
 (segment (start 152.4 48.26) (end 149.86 48.26) (width 1) (layer "F.Cu") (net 18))
 (segment (start 157.550735 43.109265) (end 152.4 48.26) (width 1) (layer "F.Cu") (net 18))
 (segment (start 151.13 45.72) (end 149.86 45.72) (width 1) (layer "F.Cu") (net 17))
 (segment (start 155.010735 41.839265) (end 151.13 45.72) (width 1) (layer "F.Cu") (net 17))
 (segment (start 155.010735 27.94) (end 155.010735 41.839265) (width 1) (layer "F.Cu") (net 17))
 (segment (start 169.164 80.518) (end 169.164 71.374) (width 1) (layer "F.Cu") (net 9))
 (segment (start 172.72 81.28) (end 169.926 81.28) (width 1) (layer "F.Cu") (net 9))
 (segment (start 169.926 81.28) (end 169.164 80.518) (width 1) (layer "F.Cu") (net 9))
 (segment (start 175.26 81.28) (end 172.72 81.28) (width 1) (layer "F.Cu") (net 9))
 (segment (start 168.91 71.12) (end 165.1 71.12) (width 1) (layer "F.Cu") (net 9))
 (segment (start 193.04 71.12) (end 193.04 81.28) (width 1) (layer "B.Cu") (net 2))
 (segment (start 193.04 53.34) (end 193.04 63.5) (width 1) (layer "B.Cu") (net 3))
 (segment (start 169.926 67.31) (end 169.926 53.594) (width 0.5) (layer "B.Cu") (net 7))
 (segment (start 165.1 68.58) (end 168.656 68.58) (width 0.5) (layer "B.Cu") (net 7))
 (segment (start 169.926 53.594) (end 170.18 53.34) (width 0.5) (layer "B.Cu") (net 7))
 (segment (start 175.26 53.34) (end 172.72 53.34) (width 1) (layer "B.Cu") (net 7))
 (segment (start 170.18 53.34) (end 172.72 53.34) (width 0.5) (layer "B.Cu") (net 7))
 (segment (start 168.656 68.58) (end 169.926 67.31) (width 0.5) (layer "B.Cu") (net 7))
 (segment (start 180.34 71.12) (end 180.34 73.406) (width 1) (layer "F.Cu") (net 1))
 (segment (start 182.88 73.66) (end 185.42 71.12) (width 1) (layer "F.Cu") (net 1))
 (segment (start 180.594 73.66) (end 182.88 73.66) (width 1) (layer "F.Cu") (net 1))
 (segment (start 180.34 73.406) (end 180.594 73.66) (width 1) (layer "F.Cu") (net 1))
 (segment (start 185.349813 81.28) (end 185.349813 71.190187) (width 1) (layer "B.Cu") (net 1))
 (segment (start 187.96 76.2) (end 185.42 76.2) (width 1) (layer "B.Cu") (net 1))
 (segment (start 185.349813 71.190187) (end 185.42 71.12) (width 1) (layer "B.Cu") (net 1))
 (segment (start 185.42 63.5) (end 185.42 53.34) (width 1) (layer "B.Cu") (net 6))
 (segment (start 185.42 63.5) (end 182.88 63.5) (width 1) (layer "B.Cu") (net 6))
 (segment (start 187.96 58.42) (end 185.42 58.42) (width 1) (layer "B.Cu") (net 6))
 (segment (start 175.26 73.66) (end 175.26 71.12) (width 1) (layer "B.Cu") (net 10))
 (segment (start 177.8 71.12) (end 175.26 71.12) (width 1) (layer "B.Cu") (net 10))
 (segment (start 180.34 63.5) (end 177.8 63.5) (width 1) (layer "B.Cu") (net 8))
 (segment (start 175.26 60.96) (end 177.8 63.5) (width 0.5) (layer "B.Cu") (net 8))
 (segment (start 161.314042 53.061958) (end 160.782 53.594) (width 0.25) (layer "B.Cu") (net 47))
 (segment (start 161.314042 50.135545) (end 161.314042 53.061958) (width 0.25) (layer "B.Cu") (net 47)))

